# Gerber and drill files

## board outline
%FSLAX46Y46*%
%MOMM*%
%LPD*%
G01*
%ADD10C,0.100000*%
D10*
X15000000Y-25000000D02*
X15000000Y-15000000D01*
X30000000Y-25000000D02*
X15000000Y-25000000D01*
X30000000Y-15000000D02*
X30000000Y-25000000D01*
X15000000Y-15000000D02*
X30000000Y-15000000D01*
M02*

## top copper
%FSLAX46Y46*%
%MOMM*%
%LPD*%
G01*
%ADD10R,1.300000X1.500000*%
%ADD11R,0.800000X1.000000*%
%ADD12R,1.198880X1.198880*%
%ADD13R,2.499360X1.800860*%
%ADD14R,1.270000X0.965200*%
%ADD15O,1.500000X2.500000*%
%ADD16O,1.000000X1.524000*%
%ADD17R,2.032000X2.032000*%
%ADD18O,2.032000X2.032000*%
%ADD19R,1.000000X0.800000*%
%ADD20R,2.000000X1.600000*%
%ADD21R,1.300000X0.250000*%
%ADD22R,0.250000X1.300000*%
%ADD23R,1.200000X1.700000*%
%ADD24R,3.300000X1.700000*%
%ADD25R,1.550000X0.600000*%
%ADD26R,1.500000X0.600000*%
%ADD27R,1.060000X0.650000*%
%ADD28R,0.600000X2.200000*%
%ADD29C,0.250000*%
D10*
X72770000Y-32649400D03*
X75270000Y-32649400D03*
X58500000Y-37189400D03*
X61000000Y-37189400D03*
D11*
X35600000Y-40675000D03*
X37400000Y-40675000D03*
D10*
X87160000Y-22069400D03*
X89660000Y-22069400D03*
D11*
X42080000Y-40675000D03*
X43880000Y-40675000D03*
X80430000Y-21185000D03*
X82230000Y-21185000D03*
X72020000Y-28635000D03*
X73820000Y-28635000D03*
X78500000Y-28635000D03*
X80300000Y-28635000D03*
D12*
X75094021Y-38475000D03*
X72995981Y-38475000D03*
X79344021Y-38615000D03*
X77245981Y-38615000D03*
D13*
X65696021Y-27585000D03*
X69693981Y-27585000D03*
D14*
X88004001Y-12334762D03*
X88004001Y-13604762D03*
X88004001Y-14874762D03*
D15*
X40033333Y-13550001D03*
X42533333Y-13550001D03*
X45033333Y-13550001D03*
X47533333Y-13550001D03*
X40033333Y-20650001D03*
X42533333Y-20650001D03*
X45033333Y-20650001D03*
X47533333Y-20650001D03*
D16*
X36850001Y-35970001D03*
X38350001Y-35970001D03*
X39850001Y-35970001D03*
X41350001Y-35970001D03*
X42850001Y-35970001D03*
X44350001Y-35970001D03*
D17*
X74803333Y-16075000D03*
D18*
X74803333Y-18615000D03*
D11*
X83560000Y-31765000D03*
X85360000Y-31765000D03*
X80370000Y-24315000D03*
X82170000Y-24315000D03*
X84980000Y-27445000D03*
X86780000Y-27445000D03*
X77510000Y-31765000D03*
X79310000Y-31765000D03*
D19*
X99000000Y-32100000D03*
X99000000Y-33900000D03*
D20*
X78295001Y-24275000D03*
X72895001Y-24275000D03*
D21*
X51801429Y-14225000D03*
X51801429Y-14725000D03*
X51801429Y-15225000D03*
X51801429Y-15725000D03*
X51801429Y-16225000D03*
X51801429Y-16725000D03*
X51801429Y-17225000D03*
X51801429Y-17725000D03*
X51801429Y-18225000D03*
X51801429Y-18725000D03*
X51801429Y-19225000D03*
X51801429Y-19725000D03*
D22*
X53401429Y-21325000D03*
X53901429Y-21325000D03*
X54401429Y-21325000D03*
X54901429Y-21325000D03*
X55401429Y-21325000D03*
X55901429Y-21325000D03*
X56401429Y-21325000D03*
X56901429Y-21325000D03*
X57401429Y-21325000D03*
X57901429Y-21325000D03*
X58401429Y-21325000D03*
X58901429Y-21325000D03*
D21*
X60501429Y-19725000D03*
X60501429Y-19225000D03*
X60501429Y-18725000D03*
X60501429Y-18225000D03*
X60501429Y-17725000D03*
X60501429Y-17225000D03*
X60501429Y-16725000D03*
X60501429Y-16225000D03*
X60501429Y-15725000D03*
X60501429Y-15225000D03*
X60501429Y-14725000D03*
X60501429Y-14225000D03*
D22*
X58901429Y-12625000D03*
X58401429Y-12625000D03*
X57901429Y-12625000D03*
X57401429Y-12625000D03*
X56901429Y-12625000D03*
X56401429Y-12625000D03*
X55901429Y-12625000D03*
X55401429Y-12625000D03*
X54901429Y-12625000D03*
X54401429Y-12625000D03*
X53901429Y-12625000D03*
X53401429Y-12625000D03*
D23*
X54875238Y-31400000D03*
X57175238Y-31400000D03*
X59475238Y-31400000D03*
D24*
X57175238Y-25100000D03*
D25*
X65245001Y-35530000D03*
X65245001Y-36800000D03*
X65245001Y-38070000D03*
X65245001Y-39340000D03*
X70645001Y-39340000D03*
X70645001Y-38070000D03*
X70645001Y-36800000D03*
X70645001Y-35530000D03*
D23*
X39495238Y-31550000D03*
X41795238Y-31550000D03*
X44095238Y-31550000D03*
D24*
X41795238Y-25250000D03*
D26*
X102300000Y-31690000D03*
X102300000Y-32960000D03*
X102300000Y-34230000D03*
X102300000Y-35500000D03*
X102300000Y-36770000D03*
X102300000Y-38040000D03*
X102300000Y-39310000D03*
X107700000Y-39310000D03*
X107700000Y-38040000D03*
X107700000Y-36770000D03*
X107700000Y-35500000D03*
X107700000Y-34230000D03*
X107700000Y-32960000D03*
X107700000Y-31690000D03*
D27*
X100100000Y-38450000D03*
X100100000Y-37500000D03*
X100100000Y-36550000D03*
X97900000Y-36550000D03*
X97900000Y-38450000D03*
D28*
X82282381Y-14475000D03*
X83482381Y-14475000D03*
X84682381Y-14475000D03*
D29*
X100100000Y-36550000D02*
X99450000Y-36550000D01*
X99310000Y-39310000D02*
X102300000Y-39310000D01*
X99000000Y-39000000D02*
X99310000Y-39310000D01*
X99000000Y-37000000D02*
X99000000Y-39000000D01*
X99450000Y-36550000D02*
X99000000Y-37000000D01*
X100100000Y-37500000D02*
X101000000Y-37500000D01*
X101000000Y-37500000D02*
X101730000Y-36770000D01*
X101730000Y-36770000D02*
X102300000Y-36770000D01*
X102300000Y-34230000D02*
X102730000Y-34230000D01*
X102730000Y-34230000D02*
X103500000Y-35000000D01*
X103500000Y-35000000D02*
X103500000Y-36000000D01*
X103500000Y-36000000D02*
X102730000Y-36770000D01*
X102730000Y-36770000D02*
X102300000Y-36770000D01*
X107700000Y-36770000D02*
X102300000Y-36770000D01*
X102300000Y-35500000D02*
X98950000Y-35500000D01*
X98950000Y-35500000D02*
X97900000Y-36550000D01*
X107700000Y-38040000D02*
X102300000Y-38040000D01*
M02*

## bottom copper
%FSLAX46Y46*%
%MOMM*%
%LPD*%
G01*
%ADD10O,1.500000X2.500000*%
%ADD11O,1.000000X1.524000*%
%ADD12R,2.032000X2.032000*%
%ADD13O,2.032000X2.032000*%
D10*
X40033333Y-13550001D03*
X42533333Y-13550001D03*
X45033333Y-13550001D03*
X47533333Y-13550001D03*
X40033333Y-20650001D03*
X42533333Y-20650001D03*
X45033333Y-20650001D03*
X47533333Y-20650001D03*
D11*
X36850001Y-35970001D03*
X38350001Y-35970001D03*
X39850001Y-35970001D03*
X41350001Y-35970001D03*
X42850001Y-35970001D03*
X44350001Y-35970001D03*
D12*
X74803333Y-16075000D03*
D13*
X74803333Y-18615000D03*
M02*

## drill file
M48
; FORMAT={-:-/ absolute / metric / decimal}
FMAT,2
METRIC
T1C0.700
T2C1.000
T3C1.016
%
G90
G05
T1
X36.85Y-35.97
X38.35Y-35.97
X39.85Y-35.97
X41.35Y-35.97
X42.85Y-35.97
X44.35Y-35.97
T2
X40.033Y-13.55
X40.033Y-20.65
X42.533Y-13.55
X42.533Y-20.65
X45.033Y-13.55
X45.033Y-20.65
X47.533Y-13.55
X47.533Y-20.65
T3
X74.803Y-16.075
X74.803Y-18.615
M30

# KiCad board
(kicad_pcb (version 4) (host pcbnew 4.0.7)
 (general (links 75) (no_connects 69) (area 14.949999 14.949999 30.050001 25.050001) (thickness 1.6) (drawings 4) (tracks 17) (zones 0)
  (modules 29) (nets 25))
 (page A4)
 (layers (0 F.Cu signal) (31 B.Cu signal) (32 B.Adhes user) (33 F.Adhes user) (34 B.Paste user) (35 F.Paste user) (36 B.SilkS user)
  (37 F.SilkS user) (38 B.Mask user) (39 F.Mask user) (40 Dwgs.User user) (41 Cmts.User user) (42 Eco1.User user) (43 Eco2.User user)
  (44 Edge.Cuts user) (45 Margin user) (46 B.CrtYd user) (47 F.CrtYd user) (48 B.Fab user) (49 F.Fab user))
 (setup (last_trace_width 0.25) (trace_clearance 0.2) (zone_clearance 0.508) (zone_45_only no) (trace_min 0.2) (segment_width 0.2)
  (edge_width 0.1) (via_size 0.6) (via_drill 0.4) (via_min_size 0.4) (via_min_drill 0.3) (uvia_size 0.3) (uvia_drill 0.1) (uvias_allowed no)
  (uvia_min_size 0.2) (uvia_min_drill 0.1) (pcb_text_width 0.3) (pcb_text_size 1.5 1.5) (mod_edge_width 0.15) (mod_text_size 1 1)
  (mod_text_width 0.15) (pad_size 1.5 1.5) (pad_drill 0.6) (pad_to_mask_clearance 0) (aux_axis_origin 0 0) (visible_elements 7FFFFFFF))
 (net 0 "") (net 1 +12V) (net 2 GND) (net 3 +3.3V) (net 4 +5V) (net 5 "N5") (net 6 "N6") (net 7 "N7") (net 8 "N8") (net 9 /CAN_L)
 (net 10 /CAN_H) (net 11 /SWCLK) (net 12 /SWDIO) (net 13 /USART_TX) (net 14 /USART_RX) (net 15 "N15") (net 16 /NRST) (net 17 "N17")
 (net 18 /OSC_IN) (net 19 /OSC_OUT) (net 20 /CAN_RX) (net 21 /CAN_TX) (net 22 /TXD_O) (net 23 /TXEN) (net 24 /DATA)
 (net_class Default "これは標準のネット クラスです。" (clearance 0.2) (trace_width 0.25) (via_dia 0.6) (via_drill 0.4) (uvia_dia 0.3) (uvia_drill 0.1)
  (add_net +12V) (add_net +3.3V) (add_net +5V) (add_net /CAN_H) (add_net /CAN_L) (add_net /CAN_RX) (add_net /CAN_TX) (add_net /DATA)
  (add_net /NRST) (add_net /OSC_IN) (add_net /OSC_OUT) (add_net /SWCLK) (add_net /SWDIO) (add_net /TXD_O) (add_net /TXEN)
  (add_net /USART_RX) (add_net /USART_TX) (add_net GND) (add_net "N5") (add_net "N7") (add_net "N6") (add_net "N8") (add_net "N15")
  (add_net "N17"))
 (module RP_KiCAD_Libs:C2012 (layer F.Cu) (at 74.02 32.6494)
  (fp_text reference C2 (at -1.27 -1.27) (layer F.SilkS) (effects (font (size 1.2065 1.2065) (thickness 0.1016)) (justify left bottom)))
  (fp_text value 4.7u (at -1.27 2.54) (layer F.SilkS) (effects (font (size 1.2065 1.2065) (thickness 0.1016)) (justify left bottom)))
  (pad 1 smd rect (at -1.25 0) (size 1.3 1.5) (layers F.Cu F.Paste F.Mask) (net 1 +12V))
  (pad 2 smd rect (at 1.25 0) (size 1.3 1.5) (layers F.Cu F.Paste F.Mask) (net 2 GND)))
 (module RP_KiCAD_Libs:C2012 (layer F.Cu) (at 59.75 37.1894)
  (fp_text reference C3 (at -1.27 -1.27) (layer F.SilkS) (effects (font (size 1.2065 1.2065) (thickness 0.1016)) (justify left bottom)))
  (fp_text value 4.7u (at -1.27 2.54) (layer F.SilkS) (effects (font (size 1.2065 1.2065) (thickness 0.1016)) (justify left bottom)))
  (pad 1 smd rect (at -1.25 0) (size 1.3 1.5) (layers F.Cu F.Paste F.Mask) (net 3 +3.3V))
  (pad 2 smd rect (at 1.25 0) (size 1.3 1.5) (layers F.Cu F.Paste F.Mask) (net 2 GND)))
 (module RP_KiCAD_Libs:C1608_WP (layer F.Cu) (at 36.5 40.675)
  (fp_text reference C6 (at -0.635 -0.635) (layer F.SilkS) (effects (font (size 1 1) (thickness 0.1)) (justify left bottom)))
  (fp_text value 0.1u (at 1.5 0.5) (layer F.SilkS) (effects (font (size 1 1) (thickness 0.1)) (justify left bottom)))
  (pad 1 smd rect (at -0.9 0) (size 0.8 1) (layers F.Cu F.Paste F.Mask) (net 2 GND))
  (pad 2 smd rect (at 0.9 0) (size 0.8 1) (layers F.Cu F.Paste F.Mask) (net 3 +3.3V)))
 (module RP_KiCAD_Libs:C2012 (layer F.Cu) (at 88.41 22.0694)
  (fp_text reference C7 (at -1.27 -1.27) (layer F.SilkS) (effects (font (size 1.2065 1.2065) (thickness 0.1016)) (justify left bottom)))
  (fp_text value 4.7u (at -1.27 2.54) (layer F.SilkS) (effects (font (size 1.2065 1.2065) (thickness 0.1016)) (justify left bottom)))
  (pad 1 smd rect (at -1.25 0) (size 1.3 1.5) (layers F.Cu F.Paste F.Mask) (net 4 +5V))
  (pad 2 smd rect (at 1.25 0) (size 1.3 1.5) (layers F.Cu F.Paste F.Mask) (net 2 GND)))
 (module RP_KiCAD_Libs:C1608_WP (layer F.Cu) (at 42.98 40.675)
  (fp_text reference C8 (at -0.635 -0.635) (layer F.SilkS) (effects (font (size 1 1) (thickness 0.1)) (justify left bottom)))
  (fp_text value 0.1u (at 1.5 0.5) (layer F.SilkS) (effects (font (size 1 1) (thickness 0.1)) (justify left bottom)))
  (pad 1 smd rect (at -0.9 0) (size 0.8 1) (layers F.Cu F.Paste F.Mask) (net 2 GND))
  (pad 2 smd rect (at 0.9 0) (size 0.8 1) (layers F.Cu F.Paste F.Mask) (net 3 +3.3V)))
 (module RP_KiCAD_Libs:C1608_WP (layer F.Cu) (at 81.33 21.185)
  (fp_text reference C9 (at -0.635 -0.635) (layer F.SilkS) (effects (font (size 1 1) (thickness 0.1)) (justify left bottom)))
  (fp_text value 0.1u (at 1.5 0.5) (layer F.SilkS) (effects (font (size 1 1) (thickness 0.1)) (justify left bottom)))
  (pad 1 smd rect (at -0.9 0) (size 0.8 1) (layers F.Cu F.Paste F.Mask) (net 2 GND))
  (pad 2 smd rect (at 0.9 0) (size 0.8 1) (layers F.Cu F.Paste F.Mask) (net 3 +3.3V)))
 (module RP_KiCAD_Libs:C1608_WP (layer F.Cu) (at 72.92 28.635)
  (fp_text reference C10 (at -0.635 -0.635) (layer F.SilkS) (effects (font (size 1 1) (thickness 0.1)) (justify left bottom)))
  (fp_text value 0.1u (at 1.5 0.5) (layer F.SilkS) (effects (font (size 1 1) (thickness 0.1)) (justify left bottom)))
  (pad 1 smd rect (at -0.9 0) (size 0.8 1) (layers F.Cu F.Paste F.Mask) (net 2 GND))
  (pad 2 smd rect (at 0.9 0) (size 0.8 1) (layers F.Cu F.Paste F.Mask) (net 3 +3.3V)))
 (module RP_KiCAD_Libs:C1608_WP (layer F.Cu) (at 79.4 28.635)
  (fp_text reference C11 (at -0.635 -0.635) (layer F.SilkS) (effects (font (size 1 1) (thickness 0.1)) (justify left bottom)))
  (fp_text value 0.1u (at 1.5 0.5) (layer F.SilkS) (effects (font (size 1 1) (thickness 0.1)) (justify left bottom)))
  (pad 1 smd rect (at -0.9 0) (size 0.8 1) (layers F.Cu F.Paste F.Mask) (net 2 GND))
  (pad 2 smd rect (at 0.9 0) (size 0.8 1) (layers F.Cu F.Paste F.Mask) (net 3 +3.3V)))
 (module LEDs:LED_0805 (layer F.Cu) (at 74.045001 38.475)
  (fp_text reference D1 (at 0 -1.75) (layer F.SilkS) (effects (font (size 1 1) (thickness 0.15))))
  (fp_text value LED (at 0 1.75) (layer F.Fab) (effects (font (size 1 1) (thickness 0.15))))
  (pad 1 smd rect (at 1.04902 0 180) (size 1.19888 1.19888) (layers F.Cu F.Paste F.Mask) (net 3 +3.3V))
  (pad 2 smd rect (at -1.04902 0 180) (size 1.19888 1.19888) (layers F.Cu F.Paste F.Mask) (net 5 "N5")))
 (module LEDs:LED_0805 (layer F.Cu) (at 78.295001 38.615)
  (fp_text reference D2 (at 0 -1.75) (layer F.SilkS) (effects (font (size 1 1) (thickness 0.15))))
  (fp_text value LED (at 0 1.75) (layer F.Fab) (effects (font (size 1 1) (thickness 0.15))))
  (pad 1 smd rect (at 1.04902 0 180) (size 1.19888 1.19888) (layers F.Cu F.Paste F.Mask))
  (pad 2 smd rect (at -1.04902 0 180) (size 1.19888 1.19888) (layers F.Cu F.Paste F.Mask) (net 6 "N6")))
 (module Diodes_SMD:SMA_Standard (layer F.Cu) (at 67.695001 27.585)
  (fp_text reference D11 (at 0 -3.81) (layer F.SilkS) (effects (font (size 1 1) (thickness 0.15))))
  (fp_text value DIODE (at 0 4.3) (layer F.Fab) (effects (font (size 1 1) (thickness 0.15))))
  (pad 1 smd rect (at -1.99898 0) (size 2.49936 1.80086) (layers F.Cu F.Paste F.Mask) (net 1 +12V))
  (pad 2 smd rect (at 1.99898 0) (size 2.49936 1.80086) (layers F.Cu F.Paste F.Mask) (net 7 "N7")))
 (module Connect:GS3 (layer F.Cu) (at 88.004001 13.604762)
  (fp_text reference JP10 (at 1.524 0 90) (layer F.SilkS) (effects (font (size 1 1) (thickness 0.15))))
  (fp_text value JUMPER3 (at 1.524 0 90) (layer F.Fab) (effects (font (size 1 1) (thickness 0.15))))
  (pad 1 smd rect (at 0 -1.27) (size 1.27 0.9652) (layers F.Cu F.Paste F.Mask) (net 4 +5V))
  (pad 2 smd rect (at 0 0) (size 1.27 0.9652) (layers F.Cu F.Paste F.Mask) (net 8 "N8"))
  (pad 3 smd rect (at 0 1.27) (size 1.27 0.9652) (layers F.Cu F.Paste F.Mask) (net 3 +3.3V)))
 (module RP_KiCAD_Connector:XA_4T (layer F.Cu) (at 40.033333 13.550001)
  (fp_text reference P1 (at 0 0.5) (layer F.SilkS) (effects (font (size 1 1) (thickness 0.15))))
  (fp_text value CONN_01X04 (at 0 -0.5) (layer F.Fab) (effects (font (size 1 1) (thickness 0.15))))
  (pad 4 thru_hole oval (at 0 0) (size 1.5 2.5) (drill 1) (layers *.Cu *.Mask F.SilkS) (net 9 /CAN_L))
  (pad 3 thru_hole oval (at 2.5 0) (size 1.5 2.5) (drill 1) (layers *.Cu *.Mask F.SilkS) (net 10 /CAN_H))
  (pad 2 thru_hole oval (at 5 0) (size 1.5 2.5) (drill 1) (layers *.Cu *.Mask F.SilkS) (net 7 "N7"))
  (pad 1 thru_hole oval (at 7.5 0) (size 1.5 2.5) (drill 1) (layers *.Cu *.Mask F.SilkS) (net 2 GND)))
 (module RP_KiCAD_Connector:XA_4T (layer F.Cu) (at 40.033333 20.650001)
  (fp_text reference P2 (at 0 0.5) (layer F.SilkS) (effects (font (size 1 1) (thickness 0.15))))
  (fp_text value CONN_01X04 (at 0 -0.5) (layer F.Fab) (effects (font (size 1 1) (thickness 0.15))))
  (pad 4 thru_hole oval (at 0 0) (size 1.5 2.5) (drill 1) (layers *.Cu *.Mask F.SilkS) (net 9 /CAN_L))
  (pad 3 thru_hole oval (at 2.5 0) (size 1.5 2.5) (drill 1) (layers *.Cu *.Mask F.SilkS) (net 10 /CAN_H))
  (pad 2 thru_hole oval (at 5 0) (size 1.5 2.5) (drill 1) (layers *.Cu *.Mask F.SilkS) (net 7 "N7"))
  (pad 1 thru_hole oval (at 7.5 0) (size 1.5 2.5) (drill 1) (layers *.Cu *.Mask F.SilkS) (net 2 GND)))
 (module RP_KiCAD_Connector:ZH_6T (layer F.Cu) (at 36.850001 35.970001)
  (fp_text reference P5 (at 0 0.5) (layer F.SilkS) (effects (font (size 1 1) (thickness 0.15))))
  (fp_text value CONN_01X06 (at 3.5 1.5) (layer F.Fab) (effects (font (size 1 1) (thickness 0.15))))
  (pad 1 thru_hole oval (at 0 0) (size 1 1.524) (drill 0.7) (layers *.Cu *.Mask) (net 2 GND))
  (pad 2 thru_hole oval (at 1.5 0) (size 1 1.524) (drill 0.7) (layers *.Cu *.Mask) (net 8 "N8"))
  (pad 3 thru_hole oval (at 3 0) (size 1 1.524) (drill 0.7) (layers *.Cu *.Mask) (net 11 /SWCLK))
  (pad 4 thru_hole oval (at 4.5 0) (size 1 1.524) (drill 0.7) (layers *.Cu *.Mask) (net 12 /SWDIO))
  (pad 5 thru_hole oval (at 6 0) (size 1 1.524) (drill 0.7) (layers *.Cu *.Mask) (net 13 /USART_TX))
  (pad 6 thru_hole oval (at 7.5 0) (size 1 1.524) (drill 0.7) (layers *.Cu *.Mask) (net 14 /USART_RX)))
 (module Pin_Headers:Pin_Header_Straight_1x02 (layer F.Cu) (at 74.803333 16.075)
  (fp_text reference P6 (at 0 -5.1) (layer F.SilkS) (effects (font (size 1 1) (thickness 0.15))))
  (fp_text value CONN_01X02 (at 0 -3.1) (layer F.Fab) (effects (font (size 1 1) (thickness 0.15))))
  (pad 1 thru_hole rect (at 0 0) (size 2.032 2.032) (drill 1.016) (layers *.Cu *.Mask F.SilkS) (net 10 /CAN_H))
  (pad 2 thru_hole oval (at 0 2.54) (size 2.032 2.032) (drill 1.016) (layers *.Cu *.Mask F.SilkS) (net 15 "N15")))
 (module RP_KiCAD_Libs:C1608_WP (layer F.Cu) (at 84.46 31.765)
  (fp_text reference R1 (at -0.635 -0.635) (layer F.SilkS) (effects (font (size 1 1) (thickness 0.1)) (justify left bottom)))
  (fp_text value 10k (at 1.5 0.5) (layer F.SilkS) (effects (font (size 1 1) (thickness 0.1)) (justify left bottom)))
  (pad 1 smd rect (at -0.9 0) (size 0.8 1) (layers F.Cu F.Paste F.Mask) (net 3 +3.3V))
  (pad 2 smd rect (at 0.9 0) (size 0.8 1) (layers F.Cu F.Paste F.Mask) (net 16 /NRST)))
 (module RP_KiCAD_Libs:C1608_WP (layer F.Cu) (at 81.27 24.315)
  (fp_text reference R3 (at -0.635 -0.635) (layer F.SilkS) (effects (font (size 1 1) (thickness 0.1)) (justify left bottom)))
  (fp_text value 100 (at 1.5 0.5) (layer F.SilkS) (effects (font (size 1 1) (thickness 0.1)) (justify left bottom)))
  (pad 1 smd rect (at -0.9 0) (size 0.8 1) (layers F.Cu F.Paste F.Mask) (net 5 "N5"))
  (pad 2 smd rect (at 0.9 0) (size 0.8 1) (layers F.Cu F.Paste F.Mask) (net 2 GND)))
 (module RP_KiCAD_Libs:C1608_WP (layer F.Cu) (at 85.88 27.445)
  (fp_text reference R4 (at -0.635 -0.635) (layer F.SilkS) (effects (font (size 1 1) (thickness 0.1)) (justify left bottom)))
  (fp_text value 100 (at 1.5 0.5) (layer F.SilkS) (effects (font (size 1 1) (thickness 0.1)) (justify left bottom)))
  (pad 1 smd rect (at -0.9 0) (size 0.8 1) (layers F.Cu F.Paste F.Mask) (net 6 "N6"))
  (pad 2 smd rect (at 0.9 0) (size 0.8 1) (layers F.Cu F.Paste F.Mask) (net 2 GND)))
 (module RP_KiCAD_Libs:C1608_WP (layer F.Cu) (at 78.41 31.765)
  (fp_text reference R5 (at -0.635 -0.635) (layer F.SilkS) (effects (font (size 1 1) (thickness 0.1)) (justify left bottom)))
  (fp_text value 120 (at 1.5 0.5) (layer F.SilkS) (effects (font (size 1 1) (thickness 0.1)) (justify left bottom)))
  (pad 1 smd rect (at -0.9 0) (size 0.8 1) (layers F.Cu F.Paste F.Mask) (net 9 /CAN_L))
  (pad 2 smd rect (at 0.9 0) (size 0.8 1) (layers F.Cu F.Paste F.Mask) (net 15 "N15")))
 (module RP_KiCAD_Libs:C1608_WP (layer F.Cu) (at 99 33 270)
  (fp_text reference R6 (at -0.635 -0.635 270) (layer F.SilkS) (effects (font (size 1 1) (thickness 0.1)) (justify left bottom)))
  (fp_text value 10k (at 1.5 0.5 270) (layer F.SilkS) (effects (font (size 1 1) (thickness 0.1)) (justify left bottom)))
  (pad 1 smd rect (at -0.9 0 270) (size 0.8 1) (layers F.Cu F.Paste F.Mask) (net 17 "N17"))
  (pad 2 smd rect (at 0.9 0 270) (size 0.8 1) (layers F.Cu F.Paste F.Mask) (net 4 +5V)))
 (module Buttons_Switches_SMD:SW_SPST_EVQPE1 (layer F.Cu) (at 75.595001 24.275)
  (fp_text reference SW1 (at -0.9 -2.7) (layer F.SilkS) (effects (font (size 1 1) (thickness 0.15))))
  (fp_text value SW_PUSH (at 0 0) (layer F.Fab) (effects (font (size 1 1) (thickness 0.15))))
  (pad 2 smd rect (at 2.7 0) (size 2 1.6) (layers F.Cu F.Paste F.Mask) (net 16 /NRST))
  (pad 1 smd rect (at -2.7 0) (size 2 1.6) (layers F.Cu F.Paste F.Mask) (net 2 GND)))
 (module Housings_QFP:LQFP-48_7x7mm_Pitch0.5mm (layer F.Cu) (at 56.151429 16.975)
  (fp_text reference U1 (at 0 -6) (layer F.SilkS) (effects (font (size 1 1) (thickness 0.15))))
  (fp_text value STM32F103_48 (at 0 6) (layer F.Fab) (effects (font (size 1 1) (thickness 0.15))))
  (pad 1 smd rect (at -4.35 -2.75) (size 1.3 0.25) (layers F.Cu F.Paste F.Mask))
  (pad 2 smd rect (at -4.35 -2.25) (size 1.3 0.25) (layers F.Cu F.Paste F.Mask))
  (pad 3 smd rect (at -4.35 -1.75) (size 1.3 0.25) (layers F.Cu F.Paste F.Mask))
  (pad 4 smd rect (at -4.35 -1.25) (size 1.3 0.25) (layers F.Cu F.Paste F.Mask))
  (pad 5 smd rect (at -4.35 -0.75) (size 1.3 0.25) (layers F.Cu F.Paste F.Mask) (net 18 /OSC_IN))
  (pad 6 smd rect (at -4.35 -0.25) (size 1.3 0.25) (layers F.Cu F.Paste F.Mask) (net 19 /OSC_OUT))
  (pad 7 smd rect (at -4.35 0.25) (size 1.3 0.25) (layers F.Cu F.Paste F.Mask) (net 16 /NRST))
  (pad 8 smd rect (at -4.35 0.75) (size 1.3 0.25) (layers F.Cu F.Paste F.Mask) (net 2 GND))
  (pad 9 smd rect (at -4.35 1.25) (size 1.3 0.25) (layers F.Cu F.Paste F.Mask) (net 3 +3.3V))
  (pad 10 smd rect (at -4.35 1.75) (size 1.3 0.25) (layers F.Cu F.Paste F.Mask))
  (pad 11 smd rect (at -4.35 2.25) (size 1.3 0.25) (layers F.Cu F.Paste F.Mask))
  (pad 12 smd rect (at -4.35 2.75) (size 1.3 0.25) (layers F.Cu F.Paste F.Mask))
  (pad 13 smd rect (at -2.75 4.35 90) (size 1.3 0.25) (layers F.Cu F.Paste F.Mask))
  (pad 14 smd rect (at -2.25 4.35 90) (size 1.3 0.25) (layers F.Cu F.Paste F.Mask))
  (pad 15 smd rect (at -1.75 4.35 90) (size 1.3 0.25) (layers F.Cu F.Paste F.Mask))
  (pad 16 smd rect (at -1.25 4.35 90) (size 1.3 0.25) (layers F.Cu F.Paste F.Mask))
  (pad 17 smd rect (at -0.75 4.35 90) (size 1.3 0.25) (layers F.Cu F.Paste F.Mask))
  (pad 18 smd rect (at -0.25 4.35 90) (size 1.3 0.25) (layers F.Cu F.Paste F.Mask))
  (pad 19 smd rect (at 0.25 4.35 90) (size 1.3 0.25) (layers F.Cu F.Paste F.Mask))
  (pad 20 smd rect (at 0.75 4.35 90) (size 1.3 0.25) (layers F.Cu F.Paste F.Mask))
  (pad 21 smd rect (at 1.25 4.35 90) (size 1.3 0.25) (layers F.Cu F.Paste F.Mask))
  (pad 22 smd rect (at 1.75 4.35 90) (size 1.3 0.25) (layers F.Cu F.Paste F.Mask))
  (pad 23 smd rect (at 2.25 4.35 90) (size 1.3 0.25) (layers F.Cu F.Paste F.Mask) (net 2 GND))
  (pad 24 smd rect (at 2.75 4.35 90) (size 1.3 0.25) (layers F.Cu F.Paste F.Mask) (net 3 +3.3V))
  (pad 25 smd rect (at 4.35 2.75) (size 1.3 0.25) (layers F.Cu F.Paste F.Mask))
  (pad 26 smd rect (at 4.35 2.25) (size 1.3 0.25) (layers F.Cu F.Paste F.Mask))
  (pad 27 smd rect (at 4.35 1.75) (size 1.3 0.25) (layers F.Cu F.Paste F.Mask))
  (pad 28 smd rect (at 4.35 1.25) (size 1.3 0.25) (layers F.Cu F.Paste F.Mask))
  (pad 29 smd rect (at 4.35 0.75) (size 1.3 0.25) (layers F.Cu F.Paste F.Mask))
  (pad 30 smd rect (at 4.35 0.25) (size 1.3 0.25) (layers F.Cu F.Paste F.Mask) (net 13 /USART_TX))
  (pad 31 smd rect (at 4.35 -0.25) (size 1.3 0.25) (layers F.Cu F.Paste F.Mask) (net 14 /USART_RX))
  (pad 32 smd rect (at 4.35 -0.75) (size 1.3 0.25) (layers F.Cu F.Paste F.Mask) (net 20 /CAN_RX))
  (pad 33 smd rect (at 4.35 -1.25) (size 1.3 0.25) (layers F.Cu F.Paste F.Mask) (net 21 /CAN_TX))
  (pad 34 smd rect (at 4.35 -1.75) (size 1.3 0.25) (layers F.Cu F.Paste F.Mask) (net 12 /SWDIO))
  (pad 35 smd rect (at 4.35 -2.25) (size 1.3 0.25) (layers F.Cu F.Paste F.Mask) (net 2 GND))
  (pad 36 smd rect (at 4.35 -2.75) (size 1.3 0.25) (layers F.Cu F.Paste F.Mask) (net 3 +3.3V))
  (pad 37 smd rect (at 2.75 -4.35 90) (size 1.3 0.25) (layers F.Cu F.Paste F.Mask) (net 11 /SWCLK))
  (pad 38 smd rect (at 2.25 -4.35 90) (size 1.3 0.25) (layers F.Cu F.Paste F.Mask))
  (pad 39 smd rect (at 1.75 -4.35 90) (size 1.3 0.25) (layers F.Cu F.Paste F.Mask))
  (pad 40 smd rect (at 1.25 -4.35 90) (size 1.3 0.25) (layers F.Cu F.Paste F.Mask))
  (pad 41 smd rect (at 0.75 -4.35 90) (size 1.3 0.25) (layers F.Cu F.Paste F.Mask))
  (pad 42 smd rect (at 0.25 -4.35 90) (size 1.3 0.25) (layers F.Cu F.Paste F.Mask))
  (pad 43 smd rect (at -0.25 -4.35 90) (size 1.3 0.25) (layers F.Cu F.Paste F.Mask))
  (pad 44 smd rect (at -0.75 -4.35 90) (size 1.3 0.25) (layers F.Cu F.Paste F.Mask))
  (pad 45 smd rect (at -1.25 -4.35 90) (size 1.3 0.25) (layers F.Cu F.Paste F.Mask))
  (pad 46 smd rect (at -1.75 -4.35 90) (size 1.3 0.25) (layers F.Cu F.Paste F.Mask))
  (pad 47 smd rect (at -2.25 -4.35 90) (size 1.3 0.25) (layers F.Cu F.Paste F.Mask) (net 2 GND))
  (pad 48 smd rect (at -2.75 -4.35 90) (size 1.3 0.25) (layers F.Cu F.Paste F.Mask) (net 3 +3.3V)))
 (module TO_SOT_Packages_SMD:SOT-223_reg (layer F.Cu) (at 57.175238 31.4)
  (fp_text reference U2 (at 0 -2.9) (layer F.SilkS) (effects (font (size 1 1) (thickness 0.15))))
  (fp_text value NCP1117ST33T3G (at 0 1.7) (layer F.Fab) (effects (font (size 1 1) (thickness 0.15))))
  (pad 1 smd rect (at -2.3 0) (size 1.2 1.7) (layers F.Cu F.Paste F.Mask) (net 2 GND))
  (pad 2 smd rect (at 0 0) (size 1.2 1.7) (layers F.Cu F.Paste F.Mask) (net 4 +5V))
  (pad 3 smd rect (at 2.3 0) (size 1.2 1.7) (layers F.Cu F.Paste F.Mask) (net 1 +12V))
  (pad 2 smd rect (at 0 -6.3) (size 3.3 1.7) (layers F.Cu F.Paste F.Mask) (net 4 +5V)))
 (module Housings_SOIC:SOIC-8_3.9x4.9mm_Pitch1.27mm (layer F.Cu) (at 67.945001 37.435)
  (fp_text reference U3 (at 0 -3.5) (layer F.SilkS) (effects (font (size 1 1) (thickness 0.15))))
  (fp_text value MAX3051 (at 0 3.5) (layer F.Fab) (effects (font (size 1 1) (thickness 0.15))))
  (pad 1 smd rect (at -2.7 -1.905) (size 1.55 0.6) (layers F.Cu F.Paste F.Mask) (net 21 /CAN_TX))
  (pad 2 smd rect (at -2.7 -0.635) (size 1.55 0.6) (layers F.Cu F.Paste F.Mask) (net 2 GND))
  (pad 3 smd rect (at -2.7 0.635) (size 1.55 0.6) (layers F.Cu F.Paste F.Mask) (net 3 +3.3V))
  (pad 4 smd rect (at -2.7 1.905) (size 1.55 0.6) (layers F.Cu F.Paste F.Mask) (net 20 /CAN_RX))
  (pad 5 smd rect (at 2.7 1.905) (size 1.55 0.6) (layers F.Cu F.Paste F.Mask) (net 2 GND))
  (pad 6 smd rect (at 2.7 0.635) (size 1.55 0.6) (layers F.Cu F.Paste F.Mask) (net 9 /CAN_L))
  (pad 7 smd rect (at 2.7 -0.635) (size 1.55 0.6) (layers F.Cu F.Paste F.Mask) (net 10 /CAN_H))
  (pad 8 smd rect (at 2.7 -1.905) (size 1.55 0.6) (layers F.Cu F.Paste F.Mask) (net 2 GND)))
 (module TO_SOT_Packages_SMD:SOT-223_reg (layer F.Cu) (at 41.795238 31.55)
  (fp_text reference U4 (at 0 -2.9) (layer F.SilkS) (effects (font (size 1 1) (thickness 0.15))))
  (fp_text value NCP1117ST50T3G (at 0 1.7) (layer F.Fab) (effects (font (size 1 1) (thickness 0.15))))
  (pad 1 smd rect (at -2.3 0) (size 1.2 1.7) (layers F.Cu F.Paste F.Mask) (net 2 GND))
  (pad 2 smd rect (at 0 0) (size 1.2 1.7) (layers F.Cu F.Paste F.Mask) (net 3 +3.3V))
  (pad 3 smd rect (at 2.3 0) (size 1.2 1.7) (layers F.Cu F.Paste F.Mask) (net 4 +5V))
  (pad 2 smd rect (at 0 -6.3) (size 3.3 1.7) (layers F.Cu F.Paste F.Mask) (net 3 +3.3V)))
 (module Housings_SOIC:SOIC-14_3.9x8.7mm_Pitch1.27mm (layer F.Cu) (at 105 35.5)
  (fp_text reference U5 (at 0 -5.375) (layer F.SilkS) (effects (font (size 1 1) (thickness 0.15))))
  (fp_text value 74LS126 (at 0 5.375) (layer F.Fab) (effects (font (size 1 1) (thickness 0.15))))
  (pad 1 smd rect (at -2.7 -3.81) (size 1.5 0.6) (layers F.Cu F.Paste F.Mask) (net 17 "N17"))
  (pad 2 smd rect (at -2.7 -2.54) (size 1.5 0.6) (layers F.Cu F.Paste F.Mask))
  (pad 3 smd rect (at -2.7 -1.27) (size 1.5 0.6) (layers F.Cu F.Paste F.Mask) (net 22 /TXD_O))
  (pad 4 smd rect (at -2.7 0) (size 1.5 0.6) (layers F.Cu F.Paste F.Mask) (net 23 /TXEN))
  (pad 5 smd rect (at -2.7 1.27) (size 1.5 0.6) (layers F.Cu F.Paste F.Mask) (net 22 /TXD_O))
  (pad 6 smd rect (at -2.7 2.54) (size 1.5 0.6) (layers F.Cu F.Paste F.Mask) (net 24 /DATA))
  (pad 7 smd rect (at -2.7 3.81) (size 1.5 0.6) (layers F.Cu F.Paste F.Mask) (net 2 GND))
  (pad 8 smd rect (at 2.7 3.81) (size 1.5 0.6) (layers F.Cu F.Paste F.Mask))
  (pad 9 smd rect (at 2.7 2.54) (size 1.5 0.6) (layers F.Cu F.Paste F.Mask) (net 24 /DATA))
  (pad 10 smd rect (at 2.7 1.27) (size 1.5 0.6) (layers F.Cu F.Paste F.Mask) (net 22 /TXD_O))
  (pad 11 smd rect (at 2.7 0) (size 1.5 0.6) (layers F.Cu F.Paste F.Mask))
  (pad 12 smd rect (at 2.7 -1.27) (size 1.5 0.6) (layers F.Cu F.Paste F.Mask))
  (pad 13 smd rect (at 2.7 -2.54) (size 1.5 0.6) (layers F.Cu F.Paste F.Mask))
  (pad 14 smd rect (at 2.7 -3.81) (size 1.5 0.6) (layers F.Cu F.Paste F.Mask)))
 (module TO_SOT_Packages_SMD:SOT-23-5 (layer F.Cu) (at 99 37.5 180)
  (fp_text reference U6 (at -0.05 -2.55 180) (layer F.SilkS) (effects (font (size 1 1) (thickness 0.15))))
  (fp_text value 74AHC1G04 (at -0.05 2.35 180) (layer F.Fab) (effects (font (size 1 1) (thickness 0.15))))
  (pad 1 smd rect (at -1.1 -0.95 180) (size 1.06 0.65) (layers F.Cu F.Paste F.Mask))
  (pad 2 smd rect (at -1.1 0 180) (size 1.06 0.65) (layers F.Cu F.Paste F.Mask) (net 22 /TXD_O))
  (pad 3 smd rect (at -1.1 0.95 180) (size 1.06 0.65) (layers F.Cu F.Paste F.Mask) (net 2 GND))
  (pad 4 smd rect (at 1.1 0.95 180) (size 1.06 0.65) (layers F.Cu F.Paste F.Mask) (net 23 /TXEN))
  (pad 5 smd rect (at 1.1 -0.95 180) (size 1.06 0.65) (layers F.Cu F.Paste F.Mask)))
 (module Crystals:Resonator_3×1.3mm (layer F.Cu) (at 83.482381 14.475)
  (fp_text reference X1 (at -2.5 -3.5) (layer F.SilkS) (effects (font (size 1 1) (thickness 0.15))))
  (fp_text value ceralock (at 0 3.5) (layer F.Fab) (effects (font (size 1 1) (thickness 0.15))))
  (pad 1 smd rect (at -1.2 0) (size 0.6 2.2) (layers F.Cu F.Paste F.Mask) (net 18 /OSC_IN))
  (pad 2 smd rect (at 0 0) (size 0.6 2.2) (layers F.Cu F.Paste F.Mask) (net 2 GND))
  (pad 3 smd rect (at 1.2 0) (size 0.6 2.2) (layers F.Cu F.Paste F.Mask) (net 19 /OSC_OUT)))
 (gr_line (start 15 25) (end 15 15) (angle 90) (layer Edge.Cuts) (width 0.1))
 (gr_line (start 30 25) (end 15 25) (angle 90) (layer Edge.Cuts) (width 0.1))
 (gr_line (start 30 15) (end 30 25) (angle 90) (layer Edge.Cuts) (width 0.1))
 (gr_line (start 15 15) (end 30 15) (angle 90) (layer Edge.Cuts) (width 0.1))
 (segment (start 100.1 36.55) (end 99.45 36.55) (width 0.25) (layer F.Cu) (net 2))
 (segment (start 99.31 39.31) (end 102.3 39.31) (width 0.25) (layer F.Cu) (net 2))
 (segment (start 99 39) (end 99.31 39.31) (width 0.25) (layer F.Cu) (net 2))
 (segment (start 99 37) (end 99 39) (width 0.25) (layer F.Cu) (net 2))
 (segment (start 99.45 36.55) (end 99 37) (width 0.25) (layer F.Cu) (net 2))
 (segment (start 100.1 37.5) (end 101 37.5) (width 0.25) (layer F.Cu) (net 22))
 (segment (start 101 37.5) (end 101.73 36.77) (width 0.25) (layer F.Cu) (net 22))
 (segment (start 101.73 36.77) (end 102.3 36.77) (width 0.25) (layer F.Cu) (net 22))
 (segment (start 102.3 34.23) (end 102.73 34.23) (width 0.25) (layer F.Cu) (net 22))
 (segment (start 102.73 34.23) (end 103.5 35) (width 0.25) (layer F.Cu) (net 22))
 (segment (start 103.5 35) (end 103.5 36) (width 0.25) (layer F.Cu) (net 22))
 (segment (start 103.5 36) (end 102.73 36.77) (width 0.25) (layer F.Cu) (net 22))
 (segment (start 102.73 36.77) (end 102.3 36.77) (width 0.25) (layer F.Cu) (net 22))
 (segment (start 107.7 36.77) (end 102.3 36.77) (width 0.25) (layer F.Cu) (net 22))
 (segment (start 102.3 35.5) (end 98.95 35.5) (width 0.25) (layer F.Cu) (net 23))
 (segment (start 98.95 35.5) (end 97.9 36.55) (width 0.25) (layer F.Cu) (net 23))
 (segment (start 107.7 38.04) (end 102.3 38.04) (width 0.25) (layer F.Cu) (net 24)))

